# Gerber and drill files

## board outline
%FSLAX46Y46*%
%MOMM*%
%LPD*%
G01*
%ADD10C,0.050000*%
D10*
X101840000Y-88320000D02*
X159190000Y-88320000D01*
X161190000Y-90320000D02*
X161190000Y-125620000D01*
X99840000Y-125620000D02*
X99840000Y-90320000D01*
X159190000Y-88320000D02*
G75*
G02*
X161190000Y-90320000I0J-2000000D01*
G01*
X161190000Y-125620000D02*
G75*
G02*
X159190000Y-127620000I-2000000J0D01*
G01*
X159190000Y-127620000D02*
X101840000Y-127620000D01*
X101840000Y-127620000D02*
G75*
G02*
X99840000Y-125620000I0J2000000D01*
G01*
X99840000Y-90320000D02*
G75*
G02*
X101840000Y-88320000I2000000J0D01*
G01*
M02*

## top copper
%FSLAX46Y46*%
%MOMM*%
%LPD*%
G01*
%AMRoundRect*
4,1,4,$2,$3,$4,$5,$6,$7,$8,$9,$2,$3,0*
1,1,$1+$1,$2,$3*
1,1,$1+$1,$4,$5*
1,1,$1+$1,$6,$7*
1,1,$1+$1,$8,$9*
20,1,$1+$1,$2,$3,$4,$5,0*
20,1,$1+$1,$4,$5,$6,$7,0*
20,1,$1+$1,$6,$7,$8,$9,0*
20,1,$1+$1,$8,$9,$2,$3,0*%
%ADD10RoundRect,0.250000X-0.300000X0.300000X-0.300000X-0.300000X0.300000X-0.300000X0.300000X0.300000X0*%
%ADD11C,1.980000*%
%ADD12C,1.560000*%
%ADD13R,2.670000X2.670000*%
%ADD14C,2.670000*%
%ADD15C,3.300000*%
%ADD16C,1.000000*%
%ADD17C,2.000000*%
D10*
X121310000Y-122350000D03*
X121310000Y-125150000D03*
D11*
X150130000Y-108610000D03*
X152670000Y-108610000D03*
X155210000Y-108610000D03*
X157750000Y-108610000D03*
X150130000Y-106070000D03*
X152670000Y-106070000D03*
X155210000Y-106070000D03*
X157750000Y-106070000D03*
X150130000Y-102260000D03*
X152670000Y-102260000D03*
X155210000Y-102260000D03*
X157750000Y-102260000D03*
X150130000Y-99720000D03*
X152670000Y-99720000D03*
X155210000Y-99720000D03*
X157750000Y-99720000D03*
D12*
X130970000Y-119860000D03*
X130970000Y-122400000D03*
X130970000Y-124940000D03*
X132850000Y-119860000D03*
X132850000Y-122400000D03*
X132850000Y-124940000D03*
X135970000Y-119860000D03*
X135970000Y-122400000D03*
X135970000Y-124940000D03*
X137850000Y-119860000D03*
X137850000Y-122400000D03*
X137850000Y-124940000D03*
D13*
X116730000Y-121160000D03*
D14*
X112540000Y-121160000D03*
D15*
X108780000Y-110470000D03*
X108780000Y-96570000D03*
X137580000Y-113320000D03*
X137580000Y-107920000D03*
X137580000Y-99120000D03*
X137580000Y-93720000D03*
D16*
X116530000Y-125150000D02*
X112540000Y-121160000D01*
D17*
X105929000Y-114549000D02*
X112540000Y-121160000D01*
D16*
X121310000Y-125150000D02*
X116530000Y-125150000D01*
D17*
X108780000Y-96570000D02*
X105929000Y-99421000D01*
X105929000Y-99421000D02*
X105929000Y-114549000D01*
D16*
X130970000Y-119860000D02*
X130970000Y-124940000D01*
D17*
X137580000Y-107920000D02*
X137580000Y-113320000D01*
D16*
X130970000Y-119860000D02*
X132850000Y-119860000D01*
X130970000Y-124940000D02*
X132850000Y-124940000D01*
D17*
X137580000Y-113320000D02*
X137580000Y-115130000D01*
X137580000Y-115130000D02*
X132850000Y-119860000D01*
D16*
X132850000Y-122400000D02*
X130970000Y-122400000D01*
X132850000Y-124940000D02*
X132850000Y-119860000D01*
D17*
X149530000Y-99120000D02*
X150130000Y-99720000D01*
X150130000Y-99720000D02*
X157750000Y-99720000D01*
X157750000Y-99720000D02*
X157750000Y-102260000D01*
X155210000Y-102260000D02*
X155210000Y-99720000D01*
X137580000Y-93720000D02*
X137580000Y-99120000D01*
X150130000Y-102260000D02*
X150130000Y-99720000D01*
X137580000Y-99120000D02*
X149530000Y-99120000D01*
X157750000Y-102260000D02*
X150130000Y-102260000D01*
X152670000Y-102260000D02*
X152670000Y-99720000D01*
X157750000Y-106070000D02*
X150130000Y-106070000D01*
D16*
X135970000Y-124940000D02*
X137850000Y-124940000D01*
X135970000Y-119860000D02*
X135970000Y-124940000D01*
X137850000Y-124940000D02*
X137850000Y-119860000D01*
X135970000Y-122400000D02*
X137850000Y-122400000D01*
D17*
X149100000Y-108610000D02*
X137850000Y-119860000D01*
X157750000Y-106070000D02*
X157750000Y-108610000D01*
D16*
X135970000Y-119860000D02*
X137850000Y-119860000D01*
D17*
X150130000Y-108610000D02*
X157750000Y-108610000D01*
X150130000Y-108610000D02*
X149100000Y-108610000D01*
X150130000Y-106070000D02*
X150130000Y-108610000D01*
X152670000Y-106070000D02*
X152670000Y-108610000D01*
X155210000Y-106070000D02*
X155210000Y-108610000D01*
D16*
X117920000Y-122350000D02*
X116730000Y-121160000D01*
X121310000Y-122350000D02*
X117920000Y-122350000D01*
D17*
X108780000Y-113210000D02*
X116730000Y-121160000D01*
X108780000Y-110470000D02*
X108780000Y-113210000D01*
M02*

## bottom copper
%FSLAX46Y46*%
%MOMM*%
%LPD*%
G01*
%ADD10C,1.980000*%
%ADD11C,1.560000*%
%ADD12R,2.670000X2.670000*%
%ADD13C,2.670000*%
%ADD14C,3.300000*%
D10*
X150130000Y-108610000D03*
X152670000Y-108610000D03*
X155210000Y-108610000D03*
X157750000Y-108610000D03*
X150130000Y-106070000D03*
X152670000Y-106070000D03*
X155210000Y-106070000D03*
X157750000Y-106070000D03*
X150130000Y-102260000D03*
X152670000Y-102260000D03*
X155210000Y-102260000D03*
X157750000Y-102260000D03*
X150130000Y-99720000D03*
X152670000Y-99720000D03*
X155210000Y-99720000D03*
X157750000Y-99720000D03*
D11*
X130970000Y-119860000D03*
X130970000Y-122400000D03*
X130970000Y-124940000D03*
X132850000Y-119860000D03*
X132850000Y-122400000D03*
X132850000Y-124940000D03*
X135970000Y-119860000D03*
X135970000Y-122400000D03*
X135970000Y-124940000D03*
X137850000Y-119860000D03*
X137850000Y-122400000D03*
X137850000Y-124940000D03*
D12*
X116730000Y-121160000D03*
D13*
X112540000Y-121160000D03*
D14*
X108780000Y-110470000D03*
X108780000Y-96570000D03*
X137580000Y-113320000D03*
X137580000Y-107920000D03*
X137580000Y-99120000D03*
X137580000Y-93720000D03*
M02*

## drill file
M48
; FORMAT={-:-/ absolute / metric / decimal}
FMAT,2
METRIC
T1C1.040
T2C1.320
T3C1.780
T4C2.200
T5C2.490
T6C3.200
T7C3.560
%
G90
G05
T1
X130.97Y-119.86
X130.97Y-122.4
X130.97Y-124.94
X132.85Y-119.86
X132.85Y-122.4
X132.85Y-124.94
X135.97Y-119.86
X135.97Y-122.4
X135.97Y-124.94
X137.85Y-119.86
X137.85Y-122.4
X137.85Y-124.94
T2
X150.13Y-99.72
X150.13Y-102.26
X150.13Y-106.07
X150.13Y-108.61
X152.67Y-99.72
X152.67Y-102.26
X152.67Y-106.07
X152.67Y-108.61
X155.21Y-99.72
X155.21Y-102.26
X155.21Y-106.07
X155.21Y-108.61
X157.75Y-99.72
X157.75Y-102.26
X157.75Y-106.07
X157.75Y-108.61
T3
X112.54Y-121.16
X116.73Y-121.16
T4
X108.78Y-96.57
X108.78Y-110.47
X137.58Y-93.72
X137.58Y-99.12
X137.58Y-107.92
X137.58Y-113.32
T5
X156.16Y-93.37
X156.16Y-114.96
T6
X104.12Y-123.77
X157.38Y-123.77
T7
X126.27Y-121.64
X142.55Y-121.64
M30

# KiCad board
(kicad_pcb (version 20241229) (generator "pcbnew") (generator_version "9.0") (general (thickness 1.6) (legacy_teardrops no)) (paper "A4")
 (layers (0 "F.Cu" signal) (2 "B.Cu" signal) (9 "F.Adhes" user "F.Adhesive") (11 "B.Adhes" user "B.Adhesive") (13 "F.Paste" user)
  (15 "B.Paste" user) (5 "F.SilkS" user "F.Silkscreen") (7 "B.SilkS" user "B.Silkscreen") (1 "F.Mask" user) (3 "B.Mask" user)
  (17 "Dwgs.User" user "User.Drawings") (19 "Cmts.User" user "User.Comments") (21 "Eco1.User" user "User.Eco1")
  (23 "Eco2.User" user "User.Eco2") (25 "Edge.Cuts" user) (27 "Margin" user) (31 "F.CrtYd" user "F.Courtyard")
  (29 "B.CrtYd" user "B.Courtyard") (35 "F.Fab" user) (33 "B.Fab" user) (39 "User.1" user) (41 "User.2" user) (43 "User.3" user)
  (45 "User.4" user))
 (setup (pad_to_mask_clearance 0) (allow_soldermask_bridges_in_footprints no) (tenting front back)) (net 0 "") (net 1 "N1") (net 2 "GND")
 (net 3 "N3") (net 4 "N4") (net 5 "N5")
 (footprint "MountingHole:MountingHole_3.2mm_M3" (layer "F.Cu") (at 104.12 123.77)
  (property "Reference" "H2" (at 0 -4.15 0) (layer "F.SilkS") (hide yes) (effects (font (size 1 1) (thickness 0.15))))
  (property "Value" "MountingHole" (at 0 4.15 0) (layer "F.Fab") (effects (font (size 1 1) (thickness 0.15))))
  (pad "" np_thru_hole circle (at 0 0) (size 3.2 3.2) (drill 3.2) (layers "*.Cu" "*.Mask")))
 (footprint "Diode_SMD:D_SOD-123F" (layer "F.Cu") (at 121.31 123.75 -90)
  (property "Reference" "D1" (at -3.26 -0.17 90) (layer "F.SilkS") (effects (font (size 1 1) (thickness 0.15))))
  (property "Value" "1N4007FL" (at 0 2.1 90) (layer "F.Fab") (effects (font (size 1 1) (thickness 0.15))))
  (pad "1" smd roundrect (at -1.4 0 270) (size 1.1 1.1) (layers "F.Cu" "F.Mask" "F.Paste") (roundrect_rratio 0.2272727273) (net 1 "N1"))
  (pad "2" smd roundrect (at 1.4 0 270) (size 1.1 1.1) (layers "F.Cu" "F.Mask" "F.Paste") (roundrect_rratio 0.2272727273) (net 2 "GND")))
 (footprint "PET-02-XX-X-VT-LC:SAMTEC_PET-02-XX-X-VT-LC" (layer "F.Cu") (at 154.16 104.31 90)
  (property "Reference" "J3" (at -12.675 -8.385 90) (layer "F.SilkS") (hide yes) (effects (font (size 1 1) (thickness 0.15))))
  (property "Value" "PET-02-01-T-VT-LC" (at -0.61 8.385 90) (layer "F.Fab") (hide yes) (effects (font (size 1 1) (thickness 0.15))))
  (pad "" np_thru_hole circle (at -10.65 2 90) (size 2.49 2.49) (drill 2.49) (layers "*.Cu" "*.Mask"))
  (pad "" np_thru_hole circle (at 10.94 2 90) (size 2.49 2.49) (drill 2.49) (layers "*.Cu" "*.Mask"))
  (pad "1" thru_hole circle (at -4.3 -4.03 90) (size 1.98 1.98) (drill 1.32) (layers "*.Cu" "*.Mask") (remove_unused_layers no) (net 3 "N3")
   (solder_mask_margin 0.102))
  (pad "1" thru_hole circle (at -4.3 -1.49 90) (size 1.98 1.98) (drill 1.32) (layers "*.Cu" "*.Mask") (remove_unused_layers no) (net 3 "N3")
   (solder_mask_margin 0.102))
  (pad "1" thru_hole circle (at -4.3 1.05 90) (size 1.98 1.98) (drill 1.32) (layers "*.Cu" "*.Mask") (remove_unused_layers no) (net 3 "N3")
   (solder_mask_margin 0.102))
  (pad "1" thru_hole circle (at -4.3 3.59 90) (size 1.98 1.98) (drill 1.32) (layers "*.Cu" "*.Mask") (remove_unused_layers no) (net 3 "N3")
   (solder_mask_margin 0.102))
  (pad "1" thru_hole circle (at -1.76 -4.03 90) (size 1.98 1.98) (drill 1.32) (layers "*.Cu" "*.Mask") (remove_unused_layers no)
   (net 3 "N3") (solder_mask_margin 0.102))
  (pad "1" thru_hole circle (at -1.76 -1.49 90) (size 1.98 1.98) (drill 1.32) (layers "*.Cu" "*.Mask") (remove_unused_layers no)
   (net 3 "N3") (solder_mask_margin 0.102))
  (pad "1" thru_hole circle (at -1.76 1.05 90) (size 1.98 1.98) (drill 1.32) (layers "*.Cu" "*.Mask") (remove_unused_layers no) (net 3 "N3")
   (solder_mask_margin 0.102))
  (pad "1" thru_hole circle (at -1.76 3.59 90) (size 1.98 1.98) (drill 1.32) (layers "*.Cu" "*.Mask") (remove_unused_layers no) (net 3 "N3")
   (solder_mask_margin 0.102))
  (pad "2" thru_hole circle (at 2.05 -4.03 90) (size 1.98 1.98) (drill 1.32) (layers "*.Cu" "*.Mask") (remove_unused_layers no) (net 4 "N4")
   (solder_mask_margin 0.102))
  (pad "2" thru_hole circle (at 2.05 -1.49 90) (size 1.98 1.98) (drill 1.32) (layers "*.Cu" "*.Mask") (remove_unused_layers no) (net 4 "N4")
   (solder_mask_margin 0.102))
  (pad "2" thru_hole circle (at 2.05 1.05 90) (size 1.98 1.98) (drill 1.32) (layers "*.Cu" "*.Mask") (remove_unused_layers no) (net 4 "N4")
   (solder_mask_margin 0.102))
  (pad "2" thru_hole circle (at 2.05 3.59 90) (size 1.98 1.98) (drill 1.32) (layers "*.Cu" "*.Mask") (remove_unused_layers no) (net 4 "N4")
   (solder_mask_margin 0.102))
  (pad "2" thru_hole circle (at 4.59 -4.03 90) (size 1.98 1.98) (drill 1.32) (layers "*.Cu" "*.Mask") (remove_unused_layers no) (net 4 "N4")
   (solder_mask_margin 0.102))
  (pad "2" thru_hole circle (at 4.59 -1.49 90) (size 1.98 1.98) (drill 1.32) (layers "*.Cu" "*.Mask") (remove_unused_layers no) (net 4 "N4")
   (solder_mask_margin 0.102))
  (pad "2" thru_hole circle (at 4.59 1.05 90) (size 1.98 1.98) (drill 1.32) (layers "*.Cu" "*.Mask") (remove_unused_layers no) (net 4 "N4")
   (solder_mask_margin 0.102))
  (pad "2" thru_hole circle (at 4.59 3.59 90) (size 1.98 1.98) (drill 1.32) (layers "*.Cu" "*.Mask") (remove_unused_layers no) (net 4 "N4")
   (solder_mask_margin 0.102)))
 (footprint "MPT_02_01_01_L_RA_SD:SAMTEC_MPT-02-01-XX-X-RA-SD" (layer "F.Cu") (at 134.41 127.79)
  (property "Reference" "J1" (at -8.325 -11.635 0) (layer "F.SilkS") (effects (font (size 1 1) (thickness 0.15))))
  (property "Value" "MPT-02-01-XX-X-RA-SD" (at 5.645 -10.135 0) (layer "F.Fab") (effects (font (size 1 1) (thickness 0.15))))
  (pad "" np_thru_hole circle (at -8.14 -6.15) (size 3.56 3.56) (drill 3.56) (layers "*.Cu" "*.Mask"))
  (pad "" np_thru_hole circle (at 8.14 -6.15) (size 3.56 3.56) (drill 3.56) (layers "*.Cu" "*.Mask"))
  (pad "1" thru_hole circle (at -3.44 -7.93) (size 1.56 1.56) (drill 1.04) (layers "*.Cu" "*.Mask") (remove_unused_layers no) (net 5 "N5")
   (solder_mask_margin 0.102))
  (pad "1" thru_hole circle (at -3.44 -5.39) (size 1.56 1.56) (drill 1.04) (layers "*.Cu" "*.Mask") (remove_unused_layers no) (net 5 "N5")
   (solder_mask_margin 0.102))
  (pad "1" thru_hole circle (at -3.44 -2.85) (size 1.56 1.56) (drill 1.04) (layers "*.Cu" "*.Mask") (remove_unused_layers no) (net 5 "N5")
   (solder_mask_margin 0.102))
  (pad "1" thru_hole circle (at -1.56 -7.93) (size 1.56 1.56) (drill 1.04) (layers "*.Cu" "*.Mask") (remove_unused_layers no) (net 5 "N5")
   (solder_mask_margin 0.102))
  (pad "1" thru_hole circle (at -1.56 -5.39) (size 1.56 1.56) (drill 1.04) (layers "*.Cu" "*.Mask") (remove_unused_layers no) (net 5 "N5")
   (solder_mask_margin 0.102))
  (pad "1" thru_hole circle (at -1.56 -2.85) (size 1.56 1.56) (drill 1.04) (layers "*.Cu" "*.Mask") (remove_unused_layers no) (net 5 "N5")
   (solder_mask_margin 0.102))
  (pad "2" thru_hole circle (at 1.56 -7.93) (size 1.56 1.56) (drill 1.04) (layers "*.Cu" "*.Mask") (remove_unused_layers no) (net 3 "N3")
   (solder_mask_margin 0.102))
  (pad "2" thru_hole circle (at 1.56 -5.39) (size 1.56 1.56) (drill 1.04) (layers "*.Cu" "*.Mask") (remove_unused_layers no) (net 3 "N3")
   (solder_mask_margin 0.102))
  (pad "2" thru_hole circle (at 1.56 -2.85) (size 1.56 1.56) (drill 1.04) (layers "*.Cu" "*.Mask") (remove_unused_layers no) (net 3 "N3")
   (solder_mask_margin 0.102))
  (pad "2" thru_hole circle (at 3.44 -7.93) (size 1.56 1.56) (drill 1.04) (layers "*.Cu" "*.Mask") (remove_unused_layers no) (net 3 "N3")
   (solder_mask_margin 0.102))
  (pad "2" thru_hole circle (at 3.44 -5.39) (size 1.56 1.56) (drill 1.04) (layers "*.Cu" "*.Mask") (remove_unused_layers no) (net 3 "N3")
   (solder_mask_margin 0.102))
  (pad "2" thru_hole circle (at 3.44 -2.85) (size 1.56 1.56) (drill 1.04) (layers "*.Cu" "*.Mask") (remove_unused_layers no) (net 3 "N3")
   (solder_mask_margin 0.102)))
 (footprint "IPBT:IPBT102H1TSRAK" (layer "F.Cu") (at 116.73 121.16 180)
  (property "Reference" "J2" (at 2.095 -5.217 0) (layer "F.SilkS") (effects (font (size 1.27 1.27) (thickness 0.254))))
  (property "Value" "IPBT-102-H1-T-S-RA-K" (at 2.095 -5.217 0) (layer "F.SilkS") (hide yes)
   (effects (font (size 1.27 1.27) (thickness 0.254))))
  (pad "1" thru_hole rect (at 0 0 180) (size 2.67 2.67) (drill 1.78) (layers "*.Cu" "*.Mask") (remove_unused_layers no) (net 1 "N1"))
  (pad "2" thru_hole circle (at 4.19 0 180) (size 2.67 2.67) (drill 1.78) (layers "*.Cu" "*.Mask") (remove_unused_layers no) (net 2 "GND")))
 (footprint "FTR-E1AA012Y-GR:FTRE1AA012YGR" (layer "F.Cu") (at 108.78 110.47)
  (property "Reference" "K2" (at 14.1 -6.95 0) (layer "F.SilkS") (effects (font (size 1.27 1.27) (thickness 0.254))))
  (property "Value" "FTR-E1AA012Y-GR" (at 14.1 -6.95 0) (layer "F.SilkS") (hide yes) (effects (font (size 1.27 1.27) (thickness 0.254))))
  (pad "1" thru_hole circle (at 0 0) (size 3.3 3.3) (drill 2.2) (layers "*.Cu" "*.Mask") (remove_unused_layers no) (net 1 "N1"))
  (pad "2" thru_hole circle (at 0 -13.9) (size 3.3 3.3) (drill 2.2) (layers "*.Cu" "*.Mask") (remove_unused_layers no) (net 2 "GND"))
  (pad "31" thru_hole circle (at 28.8 2.85) (size 3.3 3.3) (drill 2.2) (layers "*.Cu" "*.Mask") (remove_unused_layers no) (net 5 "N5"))
  (pad "32" thru_hole circle (at 28.8 -2.55) (size 3.3 3.3) (drill 2.2) (layers "*.Cu" "*.Mask") (remove_unused_layers no) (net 5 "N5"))
  (pad "41" thru_hole circle (at 28.8 -11.35) (size 3.3 3.3) (drill 2.2) (layers "*.Cu" "*.Mask") (remove_unused_layers no) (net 4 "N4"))
  (pad "42" thru_hole circle (at 28.8 -16.75) (size 3.3 3.3) (drill 2.2) (layers "*.Cu" "*.Mask") (remove_unused_layers no) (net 4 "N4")))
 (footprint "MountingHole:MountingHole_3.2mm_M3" (layer "F.Cu") (at 157.38 123.77)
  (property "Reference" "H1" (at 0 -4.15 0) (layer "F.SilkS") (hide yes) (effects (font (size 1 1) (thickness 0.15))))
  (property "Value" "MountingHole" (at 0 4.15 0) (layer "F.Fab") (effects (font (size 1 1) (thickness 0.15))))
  (pad "" np_thru_hole circle (at 0 0) (size 3.2 3.2) (drill 3.2) (layers "*.Cu" "*.Mask")))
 (gr_line (start 101.84 88.32) (end 159.19 88.32) (stroke (width 0.05) (type default)) (layer "Edge.Cuts"))
 (gr_line (start 161.19 90.32) (end 161.19 125.62) (stroke (width 0.05) (type default)) (layer "Edge.Cuts"))
 (gr_line (start 99.84 125.62) (end 99.84 90.32) (stroke (width 0.05) (type default)) (layer "Edge.Cuts"))
 (gr_arc (start 159.19 88.32) (mid 160.604214 88.905786) (end 161.19 90.32) (stroke (width 0.05) (type default)) (layer "Edge.Cuts"))
 (gr_arc (start 161.19 125.62) (mid 160.604214 127.034214) (end 159.19 127.62) (stroke (width 0.05) (type default)) (layer "Edge.Cuts"))
 (gr_line (start 159.19 127.62) (end 101.84 127.62) (stroke (width 0.05) (type default)) (layer "Edge.Cuts"))
 (gr_arc (start 101.84 127.62) (mid 100.425786 127.034214) (end 99.84 125.62) (stroke (width 0.05) (type default)) (layer "Edge.Cuts"))
 (gr_arc (start 99.84 90.32) (mid 100.425786 88.905786) (end 101.84 88.32) (stroke (width 0.05) (type default)) (layer "Edge.Cuts"))
 (segment (start 116.53 125.15) (end 112.54 121.16) (width 1) (layer "F.Cu") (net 2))
 (segment (start 105.929 114.549) (end 112.54 121.16) (width 2) (layer "F.Cu") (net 2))
 (segment (start 121.31 125.15) (end 116.53 125.15) (width 1) (layer "F.Cu") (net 2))
 (segment (start 108.78 96.57) (end 105.929 99.421) (width 2) (layer "F.Cu") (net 2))
 (segment (start 105.929 99.421) (end 105.929 114.549) (width 2) (layer "F.Cu") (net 2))
 (segment (start 130.97 119.86) (end 130.97 124.94) (width 1) (layer "F.Cu") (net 5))
 (segment (start 137.58 107.92) (end 137.58 113.32) (width 2) (layer "F.Cu") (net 5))
 (segment (start 130.97 119.86) (end 132.85 119.86) (width 1) (layer "F.Cu") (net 5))
 (segment (start 130.97 124.94) (end 132.85 124.94) (width 1) (layer "F.Cu") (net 5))
 (segment (start 137.58 113.32) (end 137.58 115.13) (width 2) (layer "F.Cu") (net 5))
 (segment (start 137.58 115.13) (end 132.85 119.86) (width 2) (layer "F.Cu") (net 5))
 (segment (start 132.85 122.4) (end 130.97 122.4) (width 1) (layer "F.Cu") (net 5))
 (segment (start 132.85 124.94) (end 132.85 119.86) (width 1) (layer "F.Cu") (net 5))
 (segment (start 149.53 99.12) (end 150.13 99.72) (width 2) (layer "F.Cu") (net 4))
 (segment (start 150.13 99.72) (end 157.75 99.72) (width 2) (layer "F.Cu") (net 4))
 (segment (start 157.75 99.72) (end 157.75 102.26) (width 2) (layer "F.Cu") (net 4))
 (segment (start 155.21 102.26) (end 155.21 99.72) (width 2) (layer "F.Cu") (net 4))
 (segment (start 137.58 93.72) (end 137.58 99.12) (width 2) (layer "F.Cu") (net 4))
 (segment (start 150.13 102.26) (end 150.13 99.72) (width 2) (layer "F.Cu") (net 4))
 (segment (start 137.58 99.12) (end 149.53 99.12) (width 2) (layer "F.Cu") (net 4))
 (segment (start 157.75 102.26) (end 150.13 102.26) (width 2) (layer "F.Cu") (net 4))
 (segment (start 152.67 102.26) (end 152.67 99.72) (width 2) (layer "F.Cu") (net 4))
 (segment (start 157.75 106.07) (end 150.13 106.07) (width 2) (layer "F.Cu") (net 3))
 (segment (start 135.97 124.94) (end 137.85 124.94) (width 1) (layer "F.Cu") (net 3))
 (segment (start 135.97 119.86) (end 135.97 124.94) (width 1) (layer "F.Cu") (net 3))
 (segment (start 137.85 124.94) (end 137.85 119.86) (width 1) (layer "F.Cu") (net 3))
 (segment (start 135.97 122.4) (end 137.85 122.4) (width 1) (layer "F.Cu") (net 3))
 (segment (start 149.1 108.61) (end 137.85 119.86) (width 2) (layer "F.Cu") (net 3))
 (segment (start 157.75 106.07) (end 157.75 108.61) (width 2) (layer "F.Cu") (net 3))
 (segment (start 135.97 119.86) (end 137.85 119.86) (width 1) (layer "F.Cu") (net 3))
 (segment (start 150.13 108.61) (end 157.75 108.61) (width 2) (layer "F.Cu") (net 3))
 (segment (start 150.13 108.61) (end 149.1 108.61) (width 2) (layer "F.Cu") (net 3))
 (segment (start 150.13 106.07) (end 150.13 108.61) (width 2) (layer "F.Cu") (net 3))
 (segment (start 152.67 106.07) (end 152.67 108.61) (width 2) (layer "F.Cu") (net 3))
 (segment (start 155.21 106.07) (end 155.21 108.61) (width 2) (layer "F.Cu") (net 3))
 (segment (start 117.92 122.35) (end 116.73 121.16) (width 1) (layer "F.Cu") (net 1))
 (segment (start 121.31 122.35) (end 117.92 122.35) (width 1) (layer "F.Cu") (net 1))
 (segment (start 108.78 113.21) (end 116.73 121.16) (width 2) (layer "F.Cu") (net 1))
 (segment (start 108.78 110.47) (end 108.78 113.21) (width 2) (layer "F.Cu") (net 1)))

